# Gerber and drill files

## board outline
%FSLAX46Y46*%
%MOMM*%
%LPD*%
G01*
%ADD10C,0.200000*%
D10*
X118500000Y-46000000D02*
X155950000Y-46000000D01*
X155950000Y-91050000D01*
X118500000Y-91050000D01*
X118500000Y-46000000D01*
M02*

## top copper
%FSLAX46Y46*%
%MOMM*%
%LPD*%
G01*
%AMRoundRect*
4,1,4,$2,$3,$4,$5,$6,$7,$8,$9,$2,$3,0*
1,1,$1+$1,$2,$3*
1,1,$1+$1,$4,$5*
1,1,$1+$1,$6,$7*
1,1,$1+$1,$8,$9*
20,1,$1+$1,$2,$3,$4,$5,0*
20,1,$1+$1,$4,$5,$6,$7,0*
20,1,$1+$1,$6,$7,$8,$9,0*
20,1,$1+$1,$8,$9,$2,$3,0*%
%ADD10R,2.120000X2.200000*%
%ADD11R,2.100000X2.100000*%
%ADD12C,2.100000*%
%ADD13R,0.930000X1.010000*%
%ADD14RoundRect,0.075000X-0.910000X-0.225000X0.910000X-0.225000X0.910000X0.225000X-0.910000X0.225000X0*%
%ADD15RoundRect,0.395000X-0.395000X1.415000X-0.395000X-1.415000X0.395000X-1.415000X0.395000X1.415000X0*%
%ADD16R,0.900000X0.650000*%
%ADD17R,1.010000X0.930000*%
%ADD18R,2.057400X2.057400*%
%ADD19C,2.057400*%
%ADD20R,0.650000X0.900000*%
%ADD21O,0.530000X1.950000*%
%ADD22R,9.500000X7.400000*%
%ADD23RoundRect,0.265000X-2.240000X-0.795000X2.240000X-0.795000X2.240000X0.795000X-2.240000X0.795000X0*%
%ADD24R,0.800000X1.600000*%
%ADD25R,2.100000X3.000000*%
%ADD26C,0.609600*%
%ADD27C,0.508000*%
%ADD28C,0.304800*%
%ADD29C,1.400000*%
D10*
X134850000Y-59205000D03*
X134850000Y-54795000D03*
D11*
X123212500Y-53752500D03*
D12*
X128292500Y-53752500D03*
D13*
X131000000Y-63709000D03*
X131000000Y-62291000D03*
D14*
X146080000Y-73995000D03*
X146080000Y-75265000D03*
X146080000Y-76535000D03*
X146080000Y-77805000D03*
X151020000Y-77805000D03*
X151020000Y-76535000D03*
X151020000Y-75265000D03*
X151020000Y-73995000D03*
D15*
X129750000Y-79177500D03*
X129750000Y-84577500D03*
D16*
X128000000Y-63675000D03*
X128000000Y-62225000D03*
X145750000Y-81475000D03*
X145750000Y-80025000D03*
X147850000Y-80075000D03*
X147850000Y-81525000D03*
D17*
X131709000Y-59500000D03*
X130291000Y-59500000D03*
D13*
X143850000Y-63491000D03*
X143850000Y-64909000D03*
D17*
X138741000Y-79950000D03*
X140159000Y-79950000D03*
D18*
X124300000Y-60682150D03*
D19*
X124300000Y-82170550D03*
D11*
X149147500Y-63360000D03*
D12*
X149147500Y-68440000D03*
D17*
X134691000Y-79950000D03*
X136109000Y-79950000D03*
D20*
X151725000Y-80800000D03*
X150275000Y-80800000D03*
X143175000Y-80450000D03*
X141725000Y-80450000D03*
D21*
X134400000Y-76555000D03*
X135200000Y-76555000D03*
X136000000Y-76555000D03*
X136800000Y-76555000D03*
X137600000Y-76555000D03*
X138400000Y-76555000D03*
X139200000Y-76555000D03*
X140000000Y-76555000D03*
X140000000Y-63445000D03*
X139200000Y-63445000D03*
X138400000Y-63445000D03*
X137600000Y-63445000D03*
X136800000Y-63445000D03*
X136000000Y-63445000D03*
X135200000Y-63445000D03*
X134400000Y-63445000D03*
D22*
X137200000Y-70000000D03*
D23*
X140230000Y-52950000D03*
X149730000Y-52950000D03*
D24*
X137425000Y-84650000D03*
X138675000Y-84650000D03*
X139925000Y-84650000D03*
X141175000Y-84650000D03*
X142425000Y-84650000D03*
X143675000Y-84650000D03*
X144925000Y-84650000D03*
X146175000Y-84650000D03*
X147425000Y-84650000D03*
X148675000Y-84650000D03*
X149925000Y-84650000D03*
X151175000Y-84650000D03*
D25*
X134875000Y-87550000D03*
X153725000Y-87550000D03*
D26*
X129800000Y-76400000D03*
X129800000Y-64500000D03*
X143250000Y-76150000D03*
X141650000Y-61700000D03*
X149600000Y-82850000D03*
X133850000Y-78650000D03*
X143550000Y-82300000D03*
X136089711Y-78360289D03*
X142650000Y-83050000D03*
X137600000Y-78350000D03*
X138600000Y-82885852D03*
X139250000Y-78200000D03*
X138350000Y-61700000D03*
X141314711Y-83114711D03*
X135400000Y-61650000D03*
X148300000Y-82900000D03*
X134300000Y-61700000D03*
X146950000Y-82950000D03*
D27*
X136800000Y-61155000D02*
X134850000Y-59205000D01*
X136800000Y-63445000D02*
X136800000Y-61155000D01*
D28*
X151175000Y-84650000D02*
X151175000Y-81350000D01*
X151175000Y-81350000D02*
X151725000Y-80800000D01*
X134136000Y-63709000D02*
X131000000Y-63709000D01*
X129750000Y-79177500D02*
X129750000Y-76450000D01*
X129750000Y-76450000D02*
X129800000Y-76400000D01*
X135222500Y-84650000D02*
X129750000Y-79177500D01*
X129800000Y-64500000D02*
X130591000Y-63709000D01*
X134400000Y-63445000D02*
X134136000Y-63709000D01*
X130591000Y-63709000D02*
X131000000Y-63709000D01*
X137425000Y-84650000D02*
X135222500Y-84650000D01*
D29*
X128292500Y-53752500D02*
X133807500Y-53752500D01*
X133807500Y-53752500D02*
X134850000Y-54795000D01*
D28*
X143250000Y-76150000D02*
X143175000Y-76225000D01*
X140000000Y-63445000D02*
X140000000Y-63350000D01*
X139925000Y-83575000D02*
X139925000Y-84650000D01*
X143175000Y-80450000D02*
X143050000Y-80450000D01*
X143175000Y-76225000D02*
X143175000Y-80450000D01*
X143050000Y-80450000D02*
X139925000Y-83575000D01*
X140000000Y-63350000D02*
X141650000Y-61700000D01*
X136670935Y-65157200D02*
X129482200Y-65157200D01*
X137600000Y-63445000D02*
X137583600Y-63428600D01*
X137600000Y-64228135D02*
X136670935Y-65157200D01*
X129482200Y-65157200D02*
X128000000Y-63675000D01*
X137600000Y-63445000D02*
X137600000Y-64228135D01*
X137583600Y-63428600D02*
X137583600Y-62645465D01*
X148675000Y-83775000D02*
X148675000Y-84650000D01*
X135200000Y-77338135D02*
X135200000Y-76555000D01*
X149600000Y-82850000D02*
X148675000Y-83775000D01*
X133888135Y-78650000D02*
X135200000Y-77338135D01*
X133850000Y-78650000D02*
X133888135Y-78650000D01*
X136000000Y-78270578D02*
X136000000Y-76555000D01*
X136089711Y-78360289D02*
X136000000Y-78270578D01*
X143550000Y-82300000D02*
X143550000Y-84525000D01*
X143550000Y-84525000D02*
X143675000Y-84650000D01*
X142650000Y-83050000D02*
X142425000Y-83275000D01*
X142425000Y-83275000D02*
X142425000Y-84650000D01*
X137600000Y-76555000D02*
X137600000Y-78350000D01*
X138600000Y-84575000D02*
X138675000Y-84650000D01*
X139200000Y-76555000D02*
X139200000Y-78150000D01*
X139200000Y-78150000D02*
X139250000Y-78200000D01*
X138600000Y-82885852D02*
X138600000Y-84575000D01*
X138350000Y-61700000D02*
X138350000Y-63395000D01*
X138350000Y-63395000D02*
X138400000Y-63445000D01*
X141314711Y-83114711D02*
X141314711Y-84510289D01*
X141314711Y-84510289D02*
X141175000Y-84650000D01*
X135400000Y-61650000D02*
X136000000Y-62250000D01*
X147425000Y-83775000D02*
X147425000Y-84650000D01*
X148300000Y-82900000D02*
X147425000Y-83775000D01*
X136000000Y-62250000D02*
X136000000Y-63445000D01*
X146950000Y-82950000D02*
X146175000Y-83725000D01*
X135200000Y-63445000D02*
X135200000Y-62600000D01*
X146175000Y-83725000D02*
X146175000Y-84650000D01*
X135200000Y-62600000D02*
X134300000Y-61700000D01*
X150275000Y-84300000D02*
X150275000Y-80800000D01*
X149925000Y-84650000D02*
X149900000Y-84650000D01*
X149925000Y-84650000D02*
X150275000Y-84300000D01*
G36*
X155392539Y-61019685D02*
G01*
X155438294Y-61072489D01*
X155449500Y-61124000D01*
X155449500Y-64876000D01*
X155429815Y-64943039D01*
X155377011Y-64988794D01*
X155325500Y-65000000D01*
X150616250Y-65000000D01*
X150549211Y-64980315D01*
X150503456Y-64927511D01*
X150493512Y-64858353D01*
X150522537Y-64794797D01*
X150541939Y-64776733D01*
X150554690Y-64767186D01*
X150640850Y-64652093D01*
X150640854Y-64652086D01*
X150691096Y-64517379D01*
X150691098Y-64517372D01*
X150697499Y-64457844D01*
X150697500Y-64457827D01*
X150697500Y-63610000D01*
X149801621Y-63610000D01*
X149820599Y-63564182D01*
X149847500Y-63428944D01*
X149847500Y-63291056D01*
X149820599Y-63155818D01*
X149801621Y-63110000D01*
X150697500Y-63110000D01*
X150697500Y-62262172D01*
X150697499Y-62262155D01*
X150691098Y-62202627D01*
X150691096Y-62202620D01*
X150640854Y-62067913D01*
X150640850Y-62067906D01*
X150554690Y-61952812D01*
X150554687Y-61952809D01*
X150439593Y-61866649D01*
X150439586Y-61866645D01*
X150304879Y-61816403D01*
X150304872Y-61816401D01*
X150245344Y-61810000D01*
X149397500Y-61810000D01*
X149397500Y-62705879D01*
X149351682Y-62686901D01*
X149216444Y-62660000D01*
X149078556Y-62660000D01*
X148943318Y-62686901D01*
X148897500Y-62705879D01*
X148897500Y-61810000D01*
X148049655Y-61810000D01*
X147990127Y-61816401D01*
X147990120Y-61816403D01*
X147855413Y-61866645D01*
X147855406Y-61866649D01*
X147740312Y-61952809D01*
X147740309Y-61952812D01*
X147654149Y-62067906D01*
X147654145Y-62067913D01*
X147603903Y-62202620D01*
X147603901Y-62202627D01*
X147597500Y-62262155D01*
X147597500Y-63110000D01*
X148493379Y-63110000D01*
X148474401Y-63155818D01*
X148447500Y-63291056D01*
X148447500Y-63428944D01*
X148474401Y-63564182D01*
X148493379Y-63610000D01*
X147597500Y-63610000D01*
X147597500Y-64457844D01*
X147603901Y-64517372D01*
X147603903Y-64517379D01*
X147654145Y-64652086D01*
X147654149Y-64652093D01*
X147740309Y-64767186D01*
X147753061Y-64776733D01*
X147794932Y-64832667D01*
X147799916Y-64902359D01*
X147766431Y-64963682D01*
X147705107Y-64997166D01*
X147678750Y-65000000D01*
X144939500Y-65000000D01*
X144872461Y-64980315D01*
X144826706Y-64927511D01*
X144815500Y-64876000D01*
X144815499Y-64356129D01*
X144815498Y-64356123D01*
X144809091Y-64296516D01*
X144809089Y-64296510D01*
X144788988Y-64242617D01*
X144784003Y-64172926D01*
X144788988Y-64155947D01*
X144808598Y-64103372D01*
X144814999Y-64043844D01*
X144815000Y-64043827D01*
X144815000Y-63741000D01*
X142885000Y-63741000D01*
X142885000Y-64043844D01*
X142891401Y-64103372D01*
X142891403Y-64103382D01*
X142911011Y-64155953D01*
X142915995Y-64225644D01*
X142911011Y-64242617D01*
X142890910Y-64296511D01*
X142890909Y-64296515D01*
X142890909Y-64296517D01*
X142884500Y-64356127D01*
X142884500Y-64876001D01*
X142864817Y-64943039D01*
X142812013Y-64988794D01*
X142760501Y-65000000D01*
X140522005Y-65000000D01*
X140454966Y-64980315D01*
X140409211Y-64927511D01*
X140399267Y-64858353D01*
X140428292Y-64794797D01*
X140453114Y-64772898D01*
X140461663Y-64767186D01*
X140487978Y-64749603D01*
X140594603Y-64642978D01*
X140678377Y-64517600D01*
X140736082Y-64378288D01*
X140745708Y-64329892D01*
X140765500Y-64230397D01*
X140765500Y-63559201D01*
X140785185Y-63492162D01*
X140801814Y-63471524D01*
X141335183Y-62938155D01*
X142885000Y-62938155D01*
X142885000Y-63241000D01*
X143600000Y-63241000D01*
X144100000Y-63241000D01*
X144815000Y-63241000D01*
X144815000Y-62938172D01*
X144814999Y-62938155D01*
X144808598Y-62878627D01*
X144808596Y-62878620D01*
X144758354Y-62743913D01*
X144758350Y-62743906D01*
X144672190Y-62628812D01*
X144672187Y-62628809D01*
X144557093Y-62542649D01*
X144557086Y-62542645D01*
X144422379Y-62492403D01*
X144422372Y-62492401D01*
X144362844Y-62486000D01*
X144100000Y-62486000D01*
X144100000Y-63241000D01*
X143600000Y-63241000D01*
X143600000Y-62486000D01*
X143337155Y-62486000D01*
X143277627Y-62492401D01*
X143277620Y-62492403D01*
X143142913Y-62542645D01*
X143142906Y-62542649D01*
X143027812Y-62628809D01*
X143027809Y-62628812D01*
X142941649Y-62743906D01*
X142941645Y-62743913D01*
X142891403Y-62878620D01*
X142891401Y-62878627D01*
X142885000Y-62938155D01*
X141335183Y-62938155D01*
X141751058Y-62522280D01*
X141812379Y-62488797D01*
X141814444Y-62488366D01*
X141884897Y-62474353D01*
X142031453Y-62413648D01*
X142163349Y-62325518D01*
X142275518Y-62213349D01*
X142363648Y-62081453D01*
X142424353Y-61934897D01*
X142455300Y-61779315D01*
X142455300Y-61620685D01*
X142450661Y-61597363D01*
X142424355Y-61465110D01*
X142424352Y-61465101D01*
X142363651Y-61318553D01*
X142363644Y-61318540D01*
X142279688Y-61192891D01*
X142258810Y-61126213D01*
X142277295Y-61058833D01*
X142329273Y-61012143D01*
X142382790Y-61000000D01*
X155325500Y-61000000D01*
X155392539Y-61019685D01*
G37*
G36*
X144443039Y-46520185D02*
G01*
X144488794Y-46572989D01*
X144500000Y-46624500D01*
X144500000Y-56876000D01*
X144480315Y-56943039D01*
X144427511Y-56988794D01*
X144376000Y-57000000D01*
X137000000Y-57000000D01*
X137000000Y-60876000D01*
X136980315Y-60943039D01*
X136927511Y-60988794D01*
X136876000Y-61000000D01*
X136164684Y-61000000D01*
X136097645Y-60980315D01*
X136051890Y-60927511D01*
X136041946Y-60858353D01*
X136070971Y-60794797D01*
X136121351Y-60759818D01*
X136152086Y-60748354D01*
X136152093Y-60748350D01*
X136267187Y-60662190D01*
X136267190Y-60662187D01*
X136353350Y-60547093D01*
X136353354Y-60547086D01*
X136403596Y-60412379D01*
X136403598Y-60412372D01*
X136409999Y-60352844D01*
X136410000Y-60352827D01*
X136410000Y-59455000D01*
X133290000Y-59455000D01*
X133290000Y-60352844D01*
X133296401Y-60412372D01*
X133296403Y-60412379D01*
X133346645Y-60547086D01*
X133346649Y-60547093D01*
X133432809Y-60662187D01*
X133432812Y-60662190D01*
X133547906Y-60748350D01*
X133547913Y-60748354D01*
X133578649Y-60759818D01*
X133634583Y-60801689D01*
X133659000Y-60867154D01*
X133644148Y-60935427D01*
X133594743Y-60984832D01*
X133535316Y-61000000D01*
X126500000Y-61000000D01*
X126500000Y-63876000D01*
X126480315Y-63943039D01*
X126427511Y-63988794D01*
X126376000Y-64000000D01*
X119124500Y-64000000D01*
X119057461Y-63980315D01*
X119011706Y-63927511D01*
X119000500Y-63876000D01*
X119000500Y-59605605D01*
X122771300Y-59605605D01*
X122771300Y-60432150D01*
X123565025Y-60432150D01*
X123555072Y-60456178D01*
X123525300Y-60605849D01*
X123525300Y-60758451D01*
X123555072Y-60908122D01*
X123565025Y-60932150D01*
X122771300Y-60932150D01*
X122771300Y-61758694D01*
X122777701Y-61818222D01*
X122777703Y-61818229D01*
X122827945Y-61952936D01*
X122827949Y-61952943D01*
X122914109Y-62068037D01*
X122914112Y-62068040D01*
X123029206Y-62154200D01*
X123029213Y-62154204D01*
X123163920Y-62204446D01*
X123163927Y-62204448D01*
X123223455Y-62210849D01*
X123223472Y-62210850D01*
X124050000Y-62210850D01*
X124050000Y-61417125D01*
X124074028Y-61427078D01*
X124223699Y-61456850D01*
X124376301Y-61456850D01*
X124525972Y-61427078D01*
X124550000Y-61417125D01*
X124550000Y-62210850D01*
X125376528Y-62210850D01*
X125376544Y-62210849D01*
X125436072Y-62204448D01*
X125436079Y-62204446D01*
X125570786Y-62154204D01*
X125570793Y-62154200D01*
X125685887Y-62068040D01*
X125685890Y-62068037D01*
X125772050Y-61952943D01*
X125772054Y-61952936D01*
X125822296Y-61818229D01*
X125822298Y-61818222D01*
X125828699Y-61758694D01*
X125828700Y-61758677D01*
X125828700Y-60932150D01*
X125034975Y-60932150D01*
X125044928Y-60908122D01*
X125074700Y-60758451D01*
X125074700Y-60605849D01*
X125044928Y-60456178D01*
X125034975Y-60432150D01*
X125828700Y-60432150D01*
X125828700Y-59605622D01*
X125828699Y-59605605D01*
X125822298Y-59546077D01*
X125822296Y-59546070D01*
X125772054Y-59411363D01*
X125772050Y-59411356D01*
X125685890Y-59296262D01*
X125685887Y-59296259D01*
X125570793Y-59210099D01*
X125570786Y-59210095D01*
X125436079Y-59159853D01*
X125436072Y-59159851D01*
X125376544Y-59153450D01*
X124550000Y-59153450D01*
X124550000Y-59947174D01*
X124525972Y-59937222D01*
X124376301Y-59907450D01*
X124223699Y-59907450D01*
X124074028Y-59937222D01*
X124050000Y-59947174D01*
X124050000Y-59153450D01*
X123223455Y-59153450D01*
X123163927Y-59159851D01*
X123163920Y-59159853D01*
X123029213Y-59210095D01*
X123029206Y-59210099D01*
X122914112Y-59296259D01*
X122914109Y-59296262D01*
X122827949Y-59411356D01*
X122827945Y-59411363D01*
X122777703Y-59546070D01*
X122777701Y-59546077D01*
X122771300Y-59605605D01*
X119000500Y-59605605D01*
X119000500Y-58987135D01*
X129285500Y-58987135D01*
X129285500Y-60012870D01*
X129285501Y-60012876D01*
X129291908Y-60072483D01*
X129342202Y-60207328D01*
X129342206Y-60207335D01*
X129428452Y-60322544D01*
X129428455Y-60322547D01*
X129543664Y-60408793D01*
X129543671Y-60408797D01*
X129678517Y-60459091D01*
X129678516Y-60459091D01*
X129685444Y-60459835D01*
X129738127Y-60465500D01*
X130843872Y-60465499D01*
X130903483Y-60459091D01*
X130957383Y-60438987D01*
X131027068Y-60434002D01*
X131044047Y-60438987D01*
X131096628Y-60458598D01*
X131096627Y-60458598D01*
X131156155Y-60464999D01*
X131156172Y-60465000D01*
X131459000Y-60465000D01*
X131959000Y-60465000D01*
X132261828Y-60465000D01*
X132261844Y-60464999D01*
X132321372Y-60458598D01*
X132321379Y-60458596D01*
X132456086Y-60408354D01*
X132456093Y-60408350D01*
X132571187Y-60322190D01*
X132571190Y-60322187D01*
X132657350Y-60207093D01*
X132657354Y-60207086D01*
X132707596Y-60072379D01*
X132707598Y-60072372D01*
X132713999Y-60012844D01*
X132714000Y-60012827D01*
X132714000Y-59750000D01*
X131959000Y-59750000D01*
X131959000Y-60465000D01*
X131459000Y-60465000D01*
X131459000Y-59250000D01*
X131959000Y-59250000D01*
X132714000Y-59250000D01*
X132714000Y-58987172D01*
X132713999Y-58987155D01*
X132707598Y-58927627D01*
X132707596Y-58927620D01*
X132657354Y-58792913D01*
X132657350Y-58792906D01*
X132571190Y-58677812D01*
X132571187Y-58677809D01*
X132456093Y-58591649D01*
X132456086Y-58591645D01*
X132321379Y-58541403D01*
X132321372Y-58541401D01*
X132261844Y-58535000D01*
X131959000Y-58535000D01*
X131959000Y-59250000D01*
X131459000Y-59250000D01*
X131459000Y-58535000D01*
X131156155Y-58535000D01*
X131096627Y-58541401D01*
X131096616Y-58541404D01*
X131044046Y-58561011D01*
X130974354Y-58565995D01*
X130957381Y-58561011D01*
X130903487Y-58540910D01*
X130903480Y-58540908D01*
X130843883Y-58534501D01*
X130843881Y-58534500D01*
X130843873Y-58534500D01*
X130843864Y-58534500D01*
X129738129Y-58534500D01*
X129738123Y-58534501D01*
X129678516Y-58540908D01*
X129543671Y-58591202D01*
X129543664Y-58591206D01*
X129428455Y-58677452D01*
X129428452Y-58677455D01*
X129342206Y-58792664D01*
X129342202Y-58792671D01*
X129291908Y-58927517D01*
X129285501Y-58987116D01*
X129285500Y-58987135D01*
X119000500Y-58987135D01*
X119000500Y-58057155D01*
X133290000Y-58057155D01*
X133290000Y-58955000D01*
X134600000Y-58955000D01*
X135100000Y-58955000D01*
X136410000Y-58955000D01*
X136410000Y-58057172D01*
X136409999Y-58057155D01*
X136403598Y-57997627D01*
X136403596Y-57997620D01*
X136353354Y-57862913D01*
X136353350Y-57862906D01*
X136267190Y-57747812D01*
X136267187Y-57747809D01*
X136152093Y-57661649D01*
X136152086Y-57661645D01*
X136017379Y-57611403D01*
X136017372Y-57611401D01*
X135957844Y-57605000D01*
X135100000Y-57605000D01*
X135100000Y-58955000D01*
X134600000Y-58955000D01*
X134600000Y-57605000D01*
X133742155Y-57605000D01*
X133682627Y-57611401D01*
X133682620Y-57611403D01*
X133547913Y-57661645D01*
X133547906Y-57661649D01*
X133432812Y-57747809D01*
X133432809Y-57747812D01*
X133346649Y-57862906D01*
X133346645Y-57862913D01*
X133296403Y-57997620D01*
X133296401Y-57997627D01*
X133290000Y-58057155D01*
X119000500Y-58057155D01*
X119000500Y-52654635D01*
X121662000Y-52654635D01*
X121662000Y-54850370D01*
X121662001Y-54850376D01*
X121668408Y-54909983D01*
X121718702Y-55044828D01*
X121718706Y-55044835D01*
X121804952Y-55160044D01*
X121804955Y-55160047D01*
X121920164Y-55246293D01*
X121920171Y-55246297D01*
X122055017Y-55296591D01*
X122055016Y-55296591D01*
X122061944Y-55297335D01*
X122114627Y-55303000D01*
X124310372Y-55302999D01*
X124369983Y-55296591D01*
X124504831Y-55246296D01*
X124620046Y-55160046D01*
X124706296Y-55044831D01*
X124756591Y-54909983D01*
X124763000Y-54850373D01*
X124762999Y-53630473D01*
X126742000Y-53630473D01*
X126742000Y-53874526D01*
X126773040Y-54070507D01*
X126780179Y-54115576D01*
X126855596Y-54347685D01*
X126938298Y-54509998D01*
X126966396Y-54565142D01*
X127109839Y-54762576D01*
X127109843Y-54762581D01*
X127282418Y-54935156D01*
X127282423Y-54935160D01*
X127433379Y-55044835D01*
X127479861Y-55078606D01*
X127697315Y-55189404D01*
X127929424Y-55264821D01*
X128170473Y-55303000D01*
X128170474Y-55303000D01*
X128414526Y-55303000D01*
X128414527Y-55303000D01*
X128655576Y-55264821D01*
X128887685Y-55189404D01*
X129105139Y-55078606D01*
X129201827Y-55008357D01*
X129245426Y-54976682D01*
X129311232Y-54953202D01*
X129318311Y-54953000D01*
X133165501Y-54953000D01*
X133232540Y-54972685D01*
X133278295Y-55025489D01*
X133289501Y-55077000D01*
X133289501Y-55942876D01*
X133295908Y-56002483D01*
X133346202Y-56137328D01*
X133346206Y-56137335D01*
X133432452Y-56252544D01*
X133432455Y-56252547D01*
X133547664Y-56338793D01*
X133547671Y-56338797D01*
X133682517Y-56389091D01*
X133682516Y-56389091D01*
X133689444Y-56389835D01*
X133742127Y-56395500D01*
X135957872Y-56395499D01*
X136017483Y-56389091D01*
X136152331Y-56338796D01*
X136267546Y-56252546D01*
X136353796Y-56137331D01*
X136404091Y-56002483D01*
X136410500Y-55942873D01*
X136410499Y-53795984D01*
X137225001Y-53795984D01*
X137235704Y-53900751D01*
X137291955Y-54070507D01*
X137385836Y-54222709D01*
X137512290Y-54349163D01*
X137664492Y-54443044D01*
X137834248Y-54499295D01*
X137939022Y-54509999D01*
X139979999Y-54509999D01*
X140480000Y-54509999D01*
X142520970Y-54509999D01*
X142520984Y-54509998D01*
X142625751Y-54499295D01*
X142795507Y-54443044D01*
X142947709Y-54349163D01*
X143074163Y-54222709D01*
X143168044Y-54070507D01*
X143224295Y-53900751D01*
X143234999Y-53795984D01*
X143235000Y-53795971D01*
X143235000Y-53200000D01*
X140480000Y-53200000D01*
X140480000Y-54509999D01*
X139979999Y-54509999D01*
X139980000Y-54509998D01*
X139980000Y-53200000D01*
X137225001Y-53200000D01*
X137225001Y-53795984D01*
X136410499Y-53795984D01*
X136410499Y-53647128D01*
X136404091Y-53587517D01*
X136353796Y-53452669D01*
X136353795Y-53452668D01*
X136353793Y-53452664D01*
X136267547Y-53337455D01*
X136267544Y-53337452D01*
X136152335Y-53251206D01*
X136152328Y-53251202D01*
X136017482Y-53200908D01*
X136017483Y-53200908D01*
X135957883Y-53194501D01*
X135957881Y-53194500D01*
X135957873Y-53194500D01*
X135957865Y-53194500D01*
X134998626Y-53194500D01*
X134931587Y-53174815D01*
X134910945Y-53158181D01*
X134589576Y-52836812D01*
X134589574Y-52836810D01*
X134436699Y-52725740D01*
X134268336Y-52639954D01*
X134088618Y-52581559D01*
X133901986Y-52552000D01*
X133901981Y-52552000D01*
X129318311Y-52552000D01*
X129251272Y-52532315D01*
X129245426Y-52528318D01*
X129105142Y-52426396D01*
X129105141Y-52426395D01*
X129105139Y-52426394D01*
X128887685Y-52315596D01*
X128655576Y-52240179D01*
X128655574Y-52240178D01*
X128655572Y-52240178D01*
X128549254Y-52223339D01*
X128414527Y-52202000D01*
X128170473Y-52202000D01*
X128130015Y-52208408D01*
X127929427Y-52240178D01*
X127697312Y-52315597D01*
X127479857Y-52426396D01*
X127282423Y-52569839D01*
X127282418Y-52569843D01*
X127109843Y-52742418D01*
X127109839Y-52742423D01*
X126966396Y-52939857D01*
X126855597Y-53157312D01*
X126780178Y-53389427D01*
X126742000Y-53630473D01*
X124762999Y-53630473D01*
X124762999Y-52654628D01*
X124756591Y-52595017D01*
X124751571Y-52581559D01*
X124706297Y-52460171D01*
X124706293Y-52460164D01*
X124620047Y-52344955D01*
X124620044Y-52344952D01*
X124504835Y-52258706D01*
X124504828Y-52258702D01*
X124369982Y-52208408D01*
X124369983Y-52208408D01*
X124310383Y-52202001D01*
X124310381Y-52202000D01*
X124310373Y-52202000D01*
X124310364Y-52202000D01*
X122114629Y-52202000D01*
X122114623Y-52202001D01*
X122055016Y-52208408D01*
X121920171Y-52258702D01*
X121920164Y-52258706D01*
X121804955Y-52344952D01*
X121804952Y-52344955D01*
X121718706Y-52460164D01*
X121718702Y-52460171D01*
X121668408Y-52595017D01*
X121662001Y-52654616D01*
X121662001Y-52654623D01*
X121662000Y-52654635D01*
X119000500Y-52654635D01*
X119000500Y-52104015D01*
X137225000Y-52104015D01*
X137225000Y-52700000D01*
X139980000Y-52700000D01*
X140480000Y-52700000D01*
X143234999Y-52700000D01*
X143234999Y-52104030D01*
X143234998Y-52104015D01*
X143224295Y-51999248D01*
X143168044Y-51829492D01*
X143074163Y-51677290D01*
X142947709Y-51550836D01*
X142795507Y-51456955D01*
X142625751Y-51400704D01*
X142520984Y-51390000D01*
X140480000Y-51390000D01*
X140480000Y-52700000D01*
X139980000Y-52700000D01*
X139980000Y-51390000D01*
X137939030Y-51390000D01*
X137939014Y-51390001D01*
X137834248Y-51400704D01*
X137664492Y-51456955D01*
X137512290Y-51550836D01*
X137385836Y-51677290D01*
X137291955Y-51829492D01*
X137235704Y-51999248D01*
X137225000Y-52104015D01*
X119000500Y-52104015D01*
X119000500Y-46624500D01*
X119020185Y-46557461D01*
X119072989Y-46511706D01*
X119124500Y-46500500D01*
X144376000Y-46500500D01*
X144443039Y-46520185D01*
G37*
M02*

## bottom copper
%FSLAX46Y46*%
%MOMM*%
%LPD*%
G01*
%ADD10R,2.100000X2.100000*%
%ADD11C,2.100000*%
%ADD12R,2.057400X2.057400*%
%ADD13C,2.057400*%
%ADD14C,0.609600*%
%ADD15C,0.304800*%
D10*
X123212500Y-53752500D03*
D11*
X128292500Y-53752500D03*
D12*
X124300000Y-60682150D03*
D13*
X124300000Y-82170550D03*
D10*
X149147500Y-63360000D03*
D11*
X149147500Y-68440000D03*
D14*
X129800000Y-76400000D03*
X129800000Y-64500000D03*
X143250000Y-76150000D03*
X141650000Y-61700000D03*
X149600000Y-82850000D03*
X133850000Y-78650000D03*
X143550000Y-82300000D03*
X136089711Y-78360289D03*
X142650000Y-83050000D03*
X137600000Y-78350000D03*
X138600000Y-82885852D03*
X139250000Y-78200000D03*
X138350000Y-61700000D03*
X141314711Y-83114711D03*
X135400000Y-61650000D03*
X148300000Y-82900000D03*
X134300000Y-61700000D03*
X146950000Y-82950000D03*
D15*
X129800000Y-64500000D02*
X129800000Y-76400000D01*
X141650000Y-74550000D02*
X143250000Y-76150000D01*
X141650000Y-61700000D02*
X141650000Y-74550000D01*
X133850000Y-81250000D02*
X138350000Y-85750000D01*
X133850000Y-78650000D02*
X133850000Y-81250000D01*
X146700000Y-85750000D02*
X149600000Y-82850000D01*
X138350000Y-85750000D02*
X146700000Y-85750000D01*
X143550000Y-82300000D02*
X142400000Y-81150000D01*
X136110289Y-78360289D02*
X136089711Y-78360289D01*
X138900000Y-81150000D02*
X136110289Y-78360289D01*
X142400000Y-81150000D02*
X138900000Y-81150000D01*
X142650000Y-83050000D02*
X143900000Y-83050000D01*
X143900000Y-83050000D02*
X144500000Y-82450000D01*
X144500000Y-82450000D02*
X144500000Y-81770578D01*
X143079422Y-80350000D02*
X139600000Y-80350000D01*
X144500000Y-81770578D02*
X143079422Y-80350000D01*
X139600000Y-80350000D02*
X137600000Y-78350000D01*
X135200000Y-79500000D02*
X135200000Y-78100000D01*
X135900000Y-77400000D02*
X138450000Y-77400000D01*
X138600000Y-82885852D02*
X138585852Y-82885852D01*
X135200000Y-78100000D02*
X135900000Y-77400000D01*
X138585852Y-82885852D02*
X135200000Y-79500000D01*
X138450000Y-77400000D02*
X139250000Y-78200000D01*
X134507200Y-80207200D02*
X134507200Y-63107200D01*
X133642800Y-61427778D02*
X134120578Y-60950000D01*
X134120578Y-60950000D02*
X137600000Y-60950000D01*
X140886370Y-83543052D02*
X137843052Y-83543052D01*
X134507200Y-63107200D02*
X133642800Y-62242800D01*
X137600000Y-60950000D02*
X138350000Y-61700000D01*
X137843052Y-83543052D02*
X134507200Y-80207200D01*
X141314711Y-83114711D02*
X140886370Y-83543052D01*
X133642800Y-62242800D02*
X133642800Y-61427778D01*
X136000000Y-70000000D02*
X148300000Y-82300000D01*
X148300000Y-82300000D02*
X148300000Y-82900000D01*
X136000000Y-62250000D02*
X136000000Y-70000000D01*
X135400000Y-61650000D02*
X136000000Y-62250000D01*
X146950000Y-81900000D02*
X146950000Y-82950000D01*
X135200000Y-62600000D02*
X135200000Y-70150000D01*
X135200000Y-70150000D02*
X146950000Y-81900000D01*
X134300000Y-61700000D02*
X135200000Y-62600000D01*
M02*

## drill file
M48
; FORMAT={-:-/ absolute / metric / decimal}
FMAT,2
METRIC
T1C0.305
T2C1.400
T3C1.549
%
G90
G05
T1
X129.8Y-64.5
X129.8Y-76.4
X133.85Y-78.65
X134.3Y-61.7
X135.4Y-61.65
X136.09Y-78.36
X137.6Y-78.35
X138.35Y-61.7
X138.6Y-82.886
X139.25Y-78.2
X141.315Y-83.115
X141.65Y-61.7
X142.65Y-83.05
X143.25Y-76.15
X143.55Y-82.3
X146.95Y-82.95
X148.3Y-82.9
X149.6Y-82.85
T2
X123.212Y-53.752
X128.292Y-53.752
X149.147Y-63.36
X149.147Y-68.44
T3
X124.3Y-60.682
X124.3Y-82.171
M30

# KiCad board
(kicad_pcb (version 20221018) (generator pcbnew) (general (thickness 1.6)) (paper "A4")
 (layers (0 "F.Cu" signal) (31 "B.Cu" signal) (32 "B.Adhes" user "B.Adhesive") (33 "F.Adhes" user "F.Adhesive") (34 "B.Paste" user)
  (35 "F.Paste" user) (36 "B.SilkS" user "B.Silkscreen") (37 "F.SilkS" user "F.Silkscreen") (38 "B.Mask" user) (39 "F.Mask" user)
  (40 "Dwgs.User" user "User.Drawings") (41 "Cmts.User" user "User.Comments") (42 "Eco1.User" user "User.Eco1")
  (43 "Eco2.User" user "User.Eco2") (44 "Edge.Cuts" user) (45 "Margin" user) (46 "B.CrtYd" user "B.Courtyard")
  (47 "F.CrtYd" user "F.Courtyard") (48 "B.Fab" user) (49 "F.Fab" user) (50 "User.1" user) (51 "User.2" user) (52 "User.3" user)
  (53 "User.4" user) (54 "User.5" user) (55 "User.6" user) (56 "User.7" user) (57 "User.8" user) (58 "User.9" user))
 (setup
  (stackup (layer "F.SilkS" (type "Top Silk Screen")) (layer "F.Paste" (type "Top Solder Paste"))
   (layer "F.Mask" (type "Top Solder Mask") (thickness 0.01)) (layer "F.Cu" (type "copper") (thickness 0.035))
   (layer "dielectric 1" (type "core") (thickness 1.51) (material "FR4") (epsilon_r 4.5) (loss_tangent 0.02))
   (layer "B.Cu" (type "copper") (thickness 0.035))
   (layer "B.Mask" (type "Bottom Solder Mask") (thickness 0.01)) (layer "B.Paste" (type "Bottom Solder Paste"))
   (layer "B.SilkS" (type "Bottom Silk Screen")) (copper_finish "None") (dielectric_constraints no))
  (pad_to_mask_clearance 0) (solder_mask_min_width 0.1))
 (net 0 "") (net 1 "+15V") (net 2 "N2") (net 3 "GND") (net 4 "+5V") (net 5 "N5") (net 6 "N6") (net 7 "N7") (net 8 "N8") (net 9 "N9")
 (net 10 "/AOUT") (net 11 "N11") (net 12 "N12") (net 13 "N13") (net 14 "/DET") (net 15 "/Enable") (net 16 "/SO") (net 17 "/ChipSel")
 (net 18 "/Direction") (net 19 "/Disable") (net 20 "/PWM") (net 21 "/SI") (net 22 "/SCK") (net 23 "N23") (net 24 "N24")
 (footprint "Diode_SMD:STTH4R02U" (layer "F.Cu") (at 134.85 57 90)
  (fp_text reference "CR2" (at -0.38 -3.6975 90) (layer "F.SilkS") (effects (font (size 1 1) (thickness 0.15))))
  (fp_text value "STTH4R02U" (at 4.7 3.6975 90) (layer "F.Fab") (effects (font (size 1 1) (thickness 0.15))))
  (pad "1" smd rect (at -2.205 0 90) (size 2.2 2.12) (layers "F.Cu" "F.Paste" "F.Mask") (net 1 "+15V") (solder_mask_margin 0.102))
  (pad "2" smd rect (at 2.205 0 90) (size 2.2 2.12) (layers "F.Cu" "F.Paste" "F.Mask") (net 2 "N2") (solder_mask_margin 0.102)))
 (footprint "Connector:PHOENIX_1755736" (layer "F.Cu") (at 119.6725 57.6225)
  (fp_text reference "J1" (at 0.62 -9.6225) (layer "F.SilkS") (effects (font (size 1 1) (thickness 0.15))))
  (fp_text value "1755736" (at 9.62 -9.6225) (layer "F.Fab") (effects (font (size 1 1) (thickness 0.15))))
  (pad "1" thru_hole rect (at 3.54 -3.87) (size 2.1 2.1) (drill 1.4) (layers "*.Cu" "*.Mask") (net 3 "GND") (solder_mask_margin 0.102))
  (pad "2" thru_hole circle (at 8.62 -3.87) (size 2.1 2.1) (drill 1.4) (layers "*.Cu" "*.Mask") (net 2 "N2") (solder_mask_margin 0.102)))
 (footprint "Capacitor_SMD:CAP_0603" (layer "F.Cu") (at 131 63 90)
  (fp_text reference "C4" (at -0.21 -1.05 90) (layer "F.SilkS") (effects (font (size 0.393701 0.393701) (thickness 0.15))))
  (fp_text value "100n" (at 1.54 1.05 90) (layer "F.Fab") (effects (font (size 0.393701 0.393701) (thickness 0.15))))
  (pad "1" smd rect (at -0.709 0 90) (size 1.01 0.93) (layers "F.Cu" "F.Paste" "F.Mask") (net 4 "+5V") (solder_mask_margin 0.102))
  (pad "2" smd rect (at 0.709 0 90) (size 1.01 0.93) (layers "F.Cu" "F.Paste" "F.Mask") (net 3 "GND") (solder_mask_margin 0.102)))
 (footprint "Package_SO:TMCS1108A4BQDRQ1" (layer "F.Cu") (at 148.55 75.9)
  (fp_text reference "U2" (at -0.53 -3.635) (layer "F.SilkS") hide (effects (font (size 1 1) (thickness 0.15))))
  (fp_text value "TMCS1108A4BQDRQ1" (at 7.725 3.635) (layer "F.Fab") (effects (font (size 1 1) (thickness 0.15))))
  (pad "1" smd roundrect (at -2.47 -1.905) (size 1.97 0.6) (layers "F.Cu" "F.Paste" "F.Mask") (roundrect_rratio 0.125) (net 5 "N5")
   (solder_mask_margin 0.102))
  (pad "2" smd roundrect (at -2.47 -0.635) (size 1.97 0.6) (layers "F.Cu" "F.Paste" "F.Mask") (roundrect_rratio 0.125) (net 5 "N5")
   (solder_mask_margin 0.102))
  (pad "3" smd roundrect (at -2.47 0.635) (size 1.97 0.6) (layers "F.Cu" "F.Paste" "F.Mask") (roundrect_rratio 0.125) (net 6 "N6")
   (solder_mask_margin 0.102))
  (pad "4" smd roundrect (at -2.47 1.905) (size 1.97 0.6) (layers "F.Cu" "F.Paste" "F.Mask") (roundrect_rratio 0.125) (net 6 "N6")
   (solder_mask_margin 0.102))
  (pad "5" smd roundrect (at 2.47 1.905) (size 1.97 0.6) (layers "F.Cu" "F.Paste" "F.Mask") (roundrect_rratio 0.125) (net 3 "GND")
   (solder_mask_margin 0.102))
  (pad "6" smd roundrect (at 2.47 0.635) (size 1.97 0.6) (layers "F.Cu" "F.Paste" "F.Mask") (roundrect_rratio 0.125) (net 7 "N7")
   (solder_mask_margin 0.102))
  (pad "7" smd roundrect (at 2.47 -0.635) (size 1.97 0.6) (layers "F.Cu" "F.Paste" "F.Mask") (roundrect_rratio 0.125) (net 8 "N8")
   (solder_mask_margin 0.102))
  (pad "8" smd roundrect (at 2.47 -1.905) (size 1.97 0.6) (layers "F.Cu" "F.Paste" "F.Mask") (roundrect_rratio 0.125) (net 4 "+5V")
   (solder_mask_margin 0.102)))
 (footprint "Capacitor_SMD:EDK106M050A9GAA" (layer "F.Cu") (at 129.75 81.8775 -90)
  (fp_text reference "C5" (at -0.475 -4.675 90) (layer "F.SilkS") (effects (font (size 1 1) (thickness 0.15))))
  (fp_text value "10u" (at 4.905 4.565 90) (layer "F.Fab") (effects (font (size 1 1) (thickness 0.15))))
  (pad "1" smd roundrect (at -2.7 0 270) (size 3.62 1.58) (layers "F.Cu" "F.Paste" "F.Mask") (roundrect_rratio 0.25) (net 4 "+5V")
   (solder_mask_margin 0.102))
  (pad "2" smd roundrect (at 2.7 0 270) (size 3.62 1.58) (layers "F.Cu" "F.Paste" "F.Mask") (roundrect_rratio 0.25) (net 3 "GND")
   (solder_mask_margin 0.102)))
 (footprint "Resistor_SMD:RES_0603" (layer "F.Cu") (at 128 62.95 90)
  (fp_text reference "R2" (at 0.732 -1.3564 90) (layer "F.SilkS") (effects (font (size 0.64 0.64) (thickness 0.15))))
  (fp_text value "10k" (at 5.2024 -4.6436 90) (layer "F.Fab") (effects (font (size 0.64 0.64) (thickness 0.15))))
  (pad "1" smd rect (at -0.725 0 90) (size 0.65 0.9) (layers "F.Cu" "F.Paste" "F.Mask") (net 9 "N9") (solder_mask_margin 0.102))
  (pad "2" smd rect (at 0.725 0 90) (size 0.65 0.9) (layers "F.Cu" "F.Paste" "F.Mask") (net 3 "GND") (solder_mask_margin 0.102)))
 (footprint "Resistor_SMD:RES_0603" (layer "F.Cu") (at 145.75 80.75 90)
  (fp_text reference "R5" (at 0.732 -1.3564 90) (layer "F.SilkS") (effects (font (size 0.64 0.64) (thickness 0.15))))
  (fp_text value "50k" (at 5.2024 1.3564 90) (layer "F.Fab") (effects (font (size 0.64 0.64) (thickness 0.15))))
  (pad "1" smd rect (at -0.725 0 90) (size 0.65 0.9) (layers "F.Cu" "F.Paste" "F.Mask") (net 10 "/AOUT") (solder_mask_margin 0.102))
  (pad "2" smd rect (at 0.725 0 90) (size 0.65 0.9) (layers "F.Cu" "F.Paste" "F.Mask") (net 3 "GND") (solder_mask_margin 0.102)))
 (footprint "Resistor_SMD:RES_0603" (layer "F.Cu") (at 147.85 80.8 -90)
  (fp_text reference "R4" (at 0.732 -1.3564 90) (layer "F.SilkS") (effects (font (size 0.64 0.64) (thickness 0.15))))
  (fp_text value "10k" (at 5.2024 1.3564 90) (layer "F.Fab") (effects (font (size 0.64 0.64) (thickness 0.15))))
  (pad "1" smd rect (at -0.725 0 270) (size 0.65 0.9) (layers "F.Cu" "F.Paste" "F.Mask") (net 8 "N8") (solder_mask_margin 0.102))
  (pad "2" smd rect (at 0.725 0 270) (size 0.65 0.9) (layers "F.Cu" "F.Paste" "F.Mask") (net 10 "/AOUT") (solder_mask_margin 0.102)))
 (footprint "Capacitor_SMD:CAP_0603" (layer "F.Cu") (at 131 59.5 180)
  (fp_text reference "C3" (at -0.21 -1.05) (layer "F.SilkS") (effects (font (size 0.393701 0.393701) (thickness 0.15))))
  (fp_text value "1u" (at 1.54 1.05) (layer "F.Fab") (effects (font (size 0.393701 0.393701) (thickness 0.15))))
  (pad "1" smd rect (at -0.709 0 180) (size 1.01 0.93) (layers "F.Cu" "F.Paste" "F.Mask") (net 1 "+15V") (solder_mask_margin 0.102))
  (pad "2" smd rect (at 0.709 0 180) (size 1.01 0.93) (layers "F.Cu" "F.Paste" "F.Mask") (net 3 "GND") (solder_mask_margin 0.102)))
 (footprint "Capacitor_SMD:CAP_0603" (layer "F.Cu") (at 143.85 64.2 -90)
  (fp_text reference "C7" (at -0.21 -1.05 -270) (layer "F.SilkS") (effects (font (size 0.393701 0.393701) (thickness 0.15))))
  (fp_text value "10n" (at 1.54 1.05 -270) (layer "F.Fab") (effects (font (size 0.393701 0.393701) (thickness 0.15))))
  (pad "1" smd rect (at -0.709 0 270) (size 1.01 0.93) (layers "F.Cu" "F.Paste" "F.Mask") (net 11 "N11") (solder_mask_margin 0.102))
  (pad "2" smd rect (at 0.709 0 270) (size 1.01 0.93) (layers "F.Cu" "F.Paste" "F.Mask") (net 3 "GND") (solder_mask_margin 0.102)))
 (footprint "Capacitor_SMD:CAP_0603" (layer "F.Cu") (at 139.45 79.95)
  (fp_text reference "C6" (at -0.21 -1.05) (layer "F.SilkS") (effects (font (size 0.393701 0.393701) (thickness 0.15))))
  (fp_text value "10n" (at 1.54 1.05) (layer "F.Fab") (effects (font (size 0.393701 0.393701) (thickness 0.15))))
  (pad "1" smd rect (at -0.709 0) (size 1.01 0.93) (layers "F.Cu" "F.Paste" "F.Mask") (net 5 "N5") (solder_mask_margin 0.102))
  (pad "2" smd rect (at 0.709 0) (size 1.01 0.93) (layers "F.Cu" "F.Paste" "F.Mask") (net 3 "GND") (solder_mask_margin 0.102)))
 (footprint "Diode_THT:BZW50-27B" (layer "F.Cu") (at 124.3 60.68215 -90)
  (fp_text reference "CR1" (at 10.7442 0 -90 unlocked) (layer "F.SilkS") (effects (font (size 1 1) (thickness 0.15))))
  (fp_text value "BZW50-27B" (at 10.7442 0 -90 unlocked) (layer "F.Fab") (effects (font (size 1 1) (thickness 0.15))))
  (pad "1" thru_hole rect (at 0 0 270) (size 2.0574 2.0574) (drill 1.5494) (layers "*.Cu" "*.Mask") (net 1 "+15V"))
  (pad "2" thru_hole circle (at 21.4884 0 270) (size 2.0574 2.0574) (drill 1.5494) (layers "*.Cu" "*.Mask") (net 3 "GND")))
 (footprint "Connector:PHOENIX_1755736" (layer "F.Cu") (at 145.2775 59.82 -90)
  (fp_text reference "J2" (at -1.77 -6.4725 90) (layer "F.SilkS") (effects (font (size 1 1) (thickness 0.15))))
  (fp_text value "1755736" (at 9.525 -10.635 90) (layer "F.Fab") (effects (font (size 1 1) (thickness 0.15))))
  (pad "1" thru_hole rect (at 3.54 -3.87 270) (size 2.1 2.1) (drill 1.4) (layers "*.Cu" "*.Mask") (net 11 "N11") (solder_mask_margin 0.102))
  (pad "2" thru_hole circle (at 8.62 -3.87 270) (size 2.1 2.1) (drill 1.4) (layers "*.Cu" "*.Mask") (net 6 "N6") (solder_mask_margin 0.102)))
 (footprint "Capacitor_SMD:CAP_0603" (layer "F.Cu") (at 135.4 79.95)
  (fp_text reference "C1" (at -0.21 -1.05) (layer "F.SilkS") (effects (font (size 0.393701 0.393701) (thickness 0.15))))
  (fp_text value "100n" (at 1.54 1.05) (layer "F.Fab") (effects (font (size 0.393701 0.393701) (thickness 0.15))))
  (pad "1" smd rect (at -0.709 0) (size 1.01 0.93) (layers "F.Cu" "F.Paste" "F.Mask") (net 1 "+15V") (solder_mask_margin 0.102))
  (pad "2" smd rect (at 0.709 0) (size 1.01 0.93) (layers "F.Cu" "F.Paste" "F.Mask") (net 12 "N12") (solder_mask_margin 0.102)))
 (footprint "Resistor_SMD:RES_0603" (layer "F.Cu") (at 151 80.8 180)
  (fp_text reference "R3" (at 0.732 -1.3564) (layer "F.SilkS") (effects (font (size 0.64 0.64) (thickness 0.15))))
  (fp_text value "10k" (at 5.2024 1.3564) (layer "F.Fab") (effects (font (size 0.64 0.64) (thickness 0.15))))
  (pad "1" smd rect (at -0.725 0 180) (size 0.65 0.9) (layers "F.Cu" "F.Paste" "F.Mask") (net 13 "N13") (solder_mask_margin 0.102))
  (pad "2" smd rect (at 0.725 0 180) (size 0.65 0.9) (layers "F.Cu" "F.Paste" "F.Mask") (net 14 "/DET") (solder_mask_margin 0.102)))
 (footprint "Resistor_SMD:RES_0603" (layer "F.Cu") (at 142.45 80.45 180)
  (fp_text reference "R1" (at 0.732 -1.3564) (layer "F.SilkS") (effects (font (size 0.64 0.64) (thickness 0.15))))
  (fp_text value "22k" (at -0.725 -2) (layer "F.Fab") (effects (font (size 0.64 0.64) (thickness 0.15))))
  (pad "1" smd rect (at -0.725 0 180) (size 0.65 0.9) (layers "F.Cu" "F.Paste" "F.Mask") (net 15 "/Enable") (solder_mask_margin 0.102))
  (pad "2" smd rect (at 0.725 0 180) (size 0.65 0.9) (layers "F.Cu" "F.Paste" "F.Mask") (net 3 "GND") (solder_mask_margin 0.102)))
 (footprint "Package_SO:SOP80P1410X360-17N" (layer "F.Cu") (at 137.2 70 90)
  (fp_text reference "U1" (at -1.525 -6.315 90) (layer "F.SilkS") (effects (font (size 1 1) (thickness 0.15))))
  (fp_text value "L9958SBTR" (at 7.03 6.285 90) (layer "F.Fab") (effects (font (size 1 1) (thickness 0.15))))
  (pad "1" smd oval (at -6.555 -2.8 90) (size 1.95 0.53) (layers "F.Cu" "F.Paste" "F.Mask") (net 3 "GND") (solder_mask_margin 0.102))
  (pad "2" smd oval (at -6.555 -2 90) (size 1.95 0.53) (layers "F.Cu" "F.Paste" "F.Mask") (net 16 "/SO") (solder_mask_margin 0.102))
  (pad "3" smd oval (at -6.555 -1.2 90) (size 1.95 0.53) (layers "F.Cu" "F.Paste" "F.Mask") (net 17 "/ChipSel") (solder_mask_margin 0.102))
  (pad "4" smd oval (at -6.555 -0.4 90) (size 1.95 0.53) (layers "F.Cu" "F.Paste" "F.Mask") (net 12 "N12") (solder_mask_margin 0.102))
  (pad "5" smd oval (at -6.555 0.4 90) (size 1.95 0.53) (layers "F.Cu" "F.Paste" "F.Mask") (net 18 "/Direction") (solder_mask_margin 0.102))
  (pad "6" smd oval (at -6.555 1.2 90) (size 1.95 0.53) (layers "F.Cu" "F.Paste" "F.Mask") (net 5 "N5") (solder_mask_margin 0.102))
  (pad "7" smd oval (at -6.555 2 90) (size 1.95 0.53) (layers "F.Cu" "F.Paste" "F.Mask") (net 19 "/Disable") (solder_mask_margin 0.102))
  (pad "8" smd oval (at -6.555 2.8 90) (size 1.95 0.53) (layers "F.Cu" "F.Paste" "F.Mask") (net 3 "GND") (solder_mask_margin 0.102))
  (pad "9" smd oval (at 6.555 2.8 90) (size 1.95 0.53) (layers "F.Cu" "F.Paste" "F.Mask") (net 15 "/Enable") (solder_mask_margin 0.102))
  (pad "10" smd oval (at 6.555 2 90) (size 1.95 0.53) (layers "F.Cu" "F.Paste" "F.Mask") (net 11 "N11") (solder_mask_margin 0.102))
  (pad "11" smd oval (at 6.555 1.2 90) (size 1.95 0.53) (layers "F.Cu" "F.Paste" "F.Mask") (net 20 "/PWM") (solder_mask_margin 0.102))
  (pad "12" smd oval (at 6.555 0.4 90) (size 1.95 0.53) (layers "F.Cu" "F.Paste" "F.Mask") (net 9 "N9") (solder_mask_margin 0.102))
  (pad "13" smd oval (at 6.555 -0.4 90) (size 1.95 0.53) (layers "F.Cu" "F.Paste" "F.Mask") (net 1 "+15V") (solder_mask_margin 0.102))
  (pad "14" smd oval (at 6.555 -1.2 90) (size 1.95 0.53) (layers "F.Cu" "F.Paste" "F.Mask") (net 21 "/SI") (solder_mask_margin 0.102))
  (pad "15" smd oval (at 6.555 -2 90) (size 1.95 0.53) (layers "F.Cu" "F.Paste" "F.Mask") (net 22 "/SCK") (solder_mask_margin 0.102))
  (pad "16" smd oval (at 6.555 -2.8 90) (size 1.95 0.53) (layers "F.Cu" "F.Paste" "F.Mask") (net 4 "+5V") (solder_mask_margin 0.102))
  (pad "17" smd rect (at 0 0 90) (size 7.4 9.5) (layers "F.Cu" "F.Mask") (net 3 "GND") (solder_mask_margin 0.102)))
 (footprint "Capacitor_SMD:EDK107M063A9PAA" (layer "F.Cu") (at 144.98 52.95)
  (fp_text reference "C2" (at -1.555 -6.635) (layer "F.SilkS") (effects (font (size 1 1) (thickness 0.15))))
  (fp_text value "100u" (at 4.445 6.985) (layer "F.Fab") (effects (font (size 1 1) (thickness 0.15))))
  (pad "1" smd roundrect (at -4.75 0) (size 5.01 2.12) (layers "F.Cu" "F.Paste" "F.Mask") (roundrect_rratio 0.125) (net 1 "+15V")
   (solder_mask_margin 0.102))
  (pad "2" smd roundrect (at 4.75 0) (size 5.01 2.12) (layers "F.Cu" "F.Paste" "F.Mask") (roundrect_rratio 0.125) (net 3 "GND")
   (solder_mask_margin 0.102)))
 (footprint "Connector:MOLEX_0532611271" (layer "F.Cu") (at 144.3 87.55)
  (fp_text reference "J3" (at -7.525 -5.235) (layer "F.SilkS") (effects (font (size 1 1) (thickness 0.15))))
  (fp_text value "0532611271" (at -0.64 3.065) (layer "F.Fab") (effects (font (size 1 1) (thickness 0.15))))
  (pad "1" smd rect (at -6.875 -2.9) (size 0.8 1.6) (layers "F.Cu" "F.Paste" "F.Mask") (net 4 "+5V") (solder_mask_margin 0.0762))
  (pad "2" smd rect (at -5.625 -2.9) (size 0.8 1.6) (layers "F.Cu" "F.Paste" "F.Mask") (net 19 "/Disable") (solder_mask_margin 0.0762))
  (pad "3" smd rect (at -4.375 -2.9) (size 0.8 1.6) (layers "F.Cu" "F.Paste" "F.Mask") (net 15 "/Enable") (solder_mask_margin 0.0762))
  (pad "4" smd rect (at -3.125 -2.9) (size 0.8 1.6) (layers "F.Cu" "F.Paste" "F.Mask") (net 20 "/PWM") (solder_mask_margin 0.0762))
  (pad "5" smd rect (at -1.875 -2.9) (size 0.8 1.6) (layers "F.Cu" "F.Paste" "F.Mask") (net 18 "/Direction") (solder_mask_margin 0.0762))
  (pad "6" smd rect (at -0.625 -2.9) (size 0.8 1.6) (layers "F.Cu" "F.Paste" "F.Mask") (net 17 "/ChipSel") (solder_mask_margin 0.0762))
  (pad "7" smd rect (at 0.625 -2.9) (size 0.8 1.6) (layers "F.Cu" "F.Paste" "F.Mask") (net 10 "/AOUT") (solder_mask_margin 0.0762))
  (pad "8" smd rect (at 1.875 -2.9) (size 0.8 1.6) (layers "F.Cu" "F.Paste" "F.Mask") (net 22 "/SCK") (solder_mask_margin 0.0762))
  (pad "9" smd rect (at 3.125 -2.9) (size 0.8 1.6) (layers "F.Cu" "F.Paste" "F.Mask") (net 21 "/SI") (solder_mask_margin 0.0762))
  (pad "10" smd rect (at 4.375 -2.9) (size 0.8 1.6) (layers "F.Cu" "F.Paste" "F.Mask") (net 16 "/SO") (solder_mask_margin 0.0762))
  (pad "11" smd rect (at 5.625 -2.9) (size 0.8 1.6) (layers "F.Cu" "F.Paste" "F.Mask") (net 14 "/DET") (solder_mask_margin 0.0762))
  (pad "12" smd rect (at 6.875 -2.9) (size 0.8 1.6) (layers "F.Cu" "F.Paste" "F.Mask") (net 13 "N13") (solder_mask_margin 0.0762))
  (pad "S1" smd rect (at -9.425 0) (size 2.1 3) (layers "F.Cu" "F.Paste" "F.Mask") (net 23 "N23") (solder_mask_margin 0.0762))
  (pad "S2" smd rect (at 9.425 0) (size 2.1 3) (layers "F.Cu" "F.Paste" "F.Mask") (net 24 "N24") (solder_mask_margin 0.0762)))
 (gr_rect (start 118.5 46) (end 155.95 91.05) (stroke (width 0.2) (type default)) (fill none) (layer "Edge.Cuts"))
 (segment (start 136.8 61.155) (end 134.85 59.205) (width 0.508) (layer "F.Cu") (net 1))
 (segment (start 136.8 63.445) (end 136.8 61.155) (width 0.508) (layer "F.Cu") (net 1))
 (segment (start 151.175 84.65) (end 151.175 81.35) (width 0.3048) (layer "F.Cu") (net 13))
 (segment (start 151.175 81.35) (end 151.725 80.8) (width 0.3048) (layer "F.Cu") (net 13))
 (segment (start 134.136 63.709) (end 131 63.709) (width 0.3048) (layer "F.Cu") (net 4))
 (segment (start 129.75 79.1775) (end 129.75 76.45) (width 0.3048) (layer "F.Cu") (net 4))
 (segment (start 129.75 76.45) (end 129.8 76.4) (width 0.3048) (layer "F.Cu") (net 4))
 (segment (start 135.2225 84.65) (end 129.75 79.1775) (width 0.3048) (layer "F.Cu") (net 4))
 (segment (start 129.8 64.5) (end 130.591 63.709) (width 0.3048) (layer "F.Cu") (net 4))
 (segment (start 134.4 63.445) (end 134.136 63.709) (width 0.3048) (layer "F.Cu") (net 4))
 (segment (start 130.591 63.709) (end 131 63.709) (width 0.3048) (layer "F.Cu") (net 4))
 (segment (start 137.425 84.65) (end 135.2225 84.65) (width 0.3048) (layer "F.Cu") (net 4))
 (via (at 129.8 76.4) (size 0.6096) (drill 0.3048) (layers "F.Cu" "B.Cu") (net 4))
 (via (at 129.8 64.5) (size 0.6096) (drill 0.3048) (layers "F.Cu" "B.Cu") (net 4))
 (segment (start 129.8 64.5) (end 129.8 76.4) (width 0.3048) (layer "B.Cu") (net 4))
 (segment (start 128.2925 53.7525) (end 133.8075 53.7525) (width 1.4) (layer "F.Cu") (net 2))
 (segment (start 133.8075 53.7525) (end 134.85 54.795) (width 1.4) (layer "F.Cu") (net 2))
 (segment (start 143.25 76.15) (end 143.175 76.225) (width 0.3048) (layer "F.Cu") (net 15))
 (segment (start 140 63.445) (end 140 63.35) (width 0.3048) (layer "F.Cu") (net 15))
 (segment (start 139.925 83.575) (end 139.925 84.65) (width 0.3048) (layer "F.Cu") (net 15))
 (segment (start 143.175 80.45) (end 143.05 80.45) (width 0.3048) (layer "F.Cu") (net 15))
 (segment (start 143.175 76.225) (end 143.175 80.45) (width 0.3048) (layer "F.Cu") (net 15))
 (segment (start 143.05 80.45) (end 139.925 83.575) (width 0.3048) (layer "F.Cu") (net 15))
 (segment (start 140 63.35) (end 141.65 61.7) (width 0.3048) (layer "F.Cu") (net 15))
 (via (at 143.25 76.15) (size 0.6096) (drill 0.3048) (layers "F.Cu" "B.Cu") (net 15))
 (via (at 141.65 61.7) (size 0.6096) (drill 0.3048) (layers "F.Cu" "B.Cu") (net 15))
 (segment (start 141.65 74.55) (end 143.25 76.15) (width 0.3048) (layer "B.Cu") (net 15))
 (segment (start 141.65 61.7) (end 141.65 74.55) (width 0.3048) (layer "B.Cu") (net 15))
 (segment (start 136.670935 65.1572) (end 129.4822 65.1572) (width 0.3048) (layer "F.Cu") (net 9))
 (segment (start 137.6 63.445) (end 137.5836 63.4286) (width 0.3048) (layer "F.Cu") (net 9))
 (segment (start 137.6 64.228135) (end 136.670935 65.1572) (width 0.3048) (layer "F.Cu") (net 9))
 (segment (start 129.4822 65.1572) (end 128 63.675) (width 0.3048) (layer "F.Cu") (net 9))
 (segment (start 137.6 63.445) (end 137.6 64.228135) (width 0.3048) (layer "F.Cu") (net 9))
 (segment (start 137.5836 63.4286) (end 137.5836 62.645465) (width 0.3048) (layer "F.Cu") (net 9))
 (segment (start 148.675 83.775) (end 148.675 84.65) (width 0.3048) (layer "F.Cu") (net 16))
 (segment (start 135.2 77.338135) (end 135.2 76.555) (width 0.3048) (layer "F.Cu") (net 16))
 (segment (start 149.6 82.85) (end 148.675 83.775) (width 0.3048) (layer "F.Cu") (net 16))
 (segment (start 133.888135 78.65) (end 135.2 77.338135) (width 0.3048) (layer "F.Cu") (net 16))
 (segment (start 133.85 78.65) (end 133.888135 78.65) (width 0.3048) (layer "F.Cu") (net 16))
 (via (at 149.6 82.85) (size 0.6096) (drill 0.3048) (layers "F.Cu" "B.Cu") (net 16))
 (via (at 133.85 78.65) (size 0.6096) (drill 0.3048) (layers "F.Cu" "B.Cu") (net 16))
 (segment (start 133.85 81.25) (end 138.35 85.75) (width 0.3048) (layer "B.Cu") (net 16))
 (segment (start 133.85 78.65) (end 133.85 81.25) (width 0.3048) (layer "B.Cu") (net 16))
 (segment (start 146.7 85.75) (end 149.6 82.85) (width 0.3048) (layer "B.Cu") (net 16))
 (segment (start 138.35 85.75) (end 146.7 85.75) (width 0.3048) (layer "B.Cu") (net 16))
 (segment (start 136 78.270578) (end 136 76.555) (width 0.3048) (layer "F.Cu") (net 17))
 (segment (start 136.089711 78.360289) (end 136 78.270578) (width 0.3048) (layer "F.Cu") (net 17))
 (segment (start 143.55 82.3) (end 143.55 84.525) (width 0.3048) (layer "F.Cu") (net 17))
 (segment (start 143.55 84.525) (end 143.675 84.65) (width 0.3048) (layer "F.Cu") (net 17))
 (via (at 143.55 82.3) (size 0.6096) (drill 0.3048) (layers "F.Cu" "B.Cu") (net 17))
 (via (at 136.089711 78.360289) (size 0.6096) (drill 0.3048) (layers "F.Cu" "B.Cu") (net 17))
 (segment (start 143.55 82.3) (end 142.4 81.15) (width 0.3048) (layer "B.Cu") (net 17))
 (segment (start 136.110289 78.360289) (end 136.089711 78.360289) (width 0.3048) (layer "B.Cu") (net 17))
 (segment (start 138.9 81.15) (end 136.110289 78.360289) (width 0.3048) (layer "B.Cu") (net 17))
 (segment (start 142.4 81.15) (end 138.9 81.15) (width 0.3048) (layer "B.Cu") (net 17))
 (segment (start 142.65 83.05) (end 142.425 83.275) (width 0.3048) (layer "F.Cu") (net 18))
 (segment (start 142.425 83.275) (end 142.425 84.65) (width 0.3048) (layer "F.Cu") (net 18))
 (segment (start 137.6 76.555) (end 137.6 78.35) (width 0.3048) (layer "F.Cu") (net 18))
 (via (at 142.65 83.05) (size 0.6096) (drill 0.3048) (layers "F.Cu" "B.Cu") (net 18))
 (via (at 137.6 78.35) (size 0.6096) (drill 0.3048) (layers "F.Cu" "B.Cu") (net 18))
 (segment (start 142.65 83.05) (end 143.9 83.05) (width 0.3048) (layer "B.Cu") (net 18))
 (segment (start 143.9 83.05) (end 144.5 82.45) (width 0.3048) (layer "B.Cu") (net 18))
 (segment (start 144.5 82.45) (end 144.5 81.770578) (width 0.3048) (layer "B.Cu") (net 18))
 (segment (start 143.079422 80.35) (end 139.6 80.35) (width 0.3048) (layer "B.Cu") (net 18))
 (segment (start 144.5 81.770578) (end 143.079422 80.35) (width 0.3048) (layer "B.Cu") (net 18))
 (segment (start 139.6 80.35) (end 137.6 78.35) (width 0.3048) (layer "B.Cu") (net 18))
 (segment (start 138.6 84.575) (end 138.675 84.65) (width 0.3048) (layer "F.Cu") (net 19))
 (segment (start 139.2 76.555) (end 139.2 78.15) (width 0.3048) (layer "F.Cu") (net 19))
 (segment (start 139.2 78.15) (end 139.25 78.2) (width 0.3048) (layer "F.Cu") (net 19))
 (segment (start 138.6 82.885852) (end 138.6 84.575) (width 0.3048) (layer "F.Cu") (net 19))
 (via (at 138.6 82.885852) (size 0.6096) (drill 0.3048) (layers "F.Cu" "B.Cu") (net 19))
 (via (at 139.25 78.2) (size 0.6096) (drill 0.3048) (layers "F.Cu" "B.Cu") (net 19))
 (segment (start 135.2 79.5) (end 135.2 78.1) (width 0.3048) (layer "B.Cu") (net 19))
 (segment (start 135.9 77.4) (end 138.45 77.4) (width 0.3048) (layer "B.Cu") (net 19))
 (segment (start 138.6 82.885852) (end 138.585852 82.885852) (width 0.3048) (layer "B.Cu") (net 19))
 (segment (start 135.2 78.1) (end 135.9 77.4) (width 0.3048) (layer "B.Cu") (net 19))
 (segment (start 138.585852 82.885852) (end 135.2 79.5) (width 0.3048) (layer "B.Cu") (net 19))
 (segment (start 138.45 77.4) (end 139.25 78.2) (width 0.3048) (layer "B.Cu") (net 19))
 (segment (start 138.35 61.7) (end 138.35 63.395) (width 0.3048) (layer "F.Cu") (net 20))
 (segment (start 138.35 63.395) (end 138.4 63.445) (width 0.3048) (layer "F.Cu") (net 20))
 (segment (start 141.314711 83.114711) (end 141.314711 84.510289) (width 0.3048) (layer "F.Cu") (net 20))
 (segment (start 141.314711 84.510289) (end 141.175 84.65) (width 0.3048) (layer "F.Cu") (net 20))
 (via (at 138.35 61.7) (size 0.6096) (drill 0.3048) (layers "F.Cu" "B.Cu") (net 20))
 (via (at 141.314711 83.114711) (size 0.6096) (drill 0.3048) (layers "F.Cu" "B.Cu") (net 20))
 (segment (start 134.5072 80.2072) (end 134.5072 63.1072) (width 0.3048) (layer "B.Cu") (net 20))
 (segment (start 133.6428 61.427778) (end 134.120578 60.95) (width 0.3048) (layer "B.Cu") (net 20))
 (segment (start 134.120578 60.95) (end 137.6 60.95) (width 0.3048) (layer "B.Cu") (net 20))
 (segment (start 140.88637 83.543052) (end 137.843052 83.543052) (width 0.3048) (layer "B.Cu") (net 20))
 (segment (start 134.5072 63.1072) (end 133.6428 62.2428) (width 0.3048) (layer "B.Cu") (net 20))
 (segment (start 137.6 60.95) (end 138.35 61.7) (width 0.3048) (layer "B.Cu") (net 20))
 (segment (start 137.843052 83.543052) (end 134.5072 80.2072) (width 0.3048) (layer "B.Cu") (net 20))
 (segment (start 141.314711 83.114711) (end 140.88637 83.543052) (width 0.3048) (layer "B.Cu") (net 20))
 (segment (start 133.6428 62.2428) (end 133.6428 61.427778) (width 0.3048) (layer "B.Cu") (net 20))
 (segment (start 135.4 61.65) (end 136 62.25) (width 0.3048) (layer "F.Cu") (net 21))
 (segment (start 147.425 83.775) (end 147.425 84.65) (width 0.3048) (layer "F.Cu") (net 21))
 (segment (start 148.3 82.9) (end 147.425 83.775) (width 0.3048) (layer "F.Cu") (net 21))
 (segment (start 136 62.25) (end 136 63.445) (width 0.3048) (layer "F.Cu") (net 21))
 (via (at 135.4 61.65) (size 0.6096) (drill 0.3048) (layers "F.Cu" "B.Cu") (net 21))
 (via (at 148.3 82.9) (size 0.6096) (drill 0.3048) (layers "F.Cu" "B.Cu") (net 21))
 (segment (start 136 70) (end 148.3 82.3) (width 0.3048) (layer "B.Cu") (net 21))
 (segment (start 148.3 82.3) (end 148.3 82.9) (width 0.3048) (layer "B.Cu") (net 21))
 (segment (start 136 62.25) (end 136 70) (width 0.3048) (layer "B.Cu") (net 21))
 (segment (start 135.4 61.65) (end 136 62.25) (width 0.3048) (layer "B.Cu") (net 21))
 (segment (start 146.95 82.95) (end 146.175 83.725) (width 0.3048) (layer "F.Cu") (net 22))
 (segment (start 135.2 63.445) (end 135.2 62.6) (width 0.3048) (layer "F.Cu") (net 22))
 (segment (start 146.175 83.725) (end 146.175 84.65) (width 0.3048) (layer "F.Cu") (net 22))
 (segment (start 135.2 62.6) (end 134.3 61.7) (width 0.3048) (layer "F.Cu") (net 22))
 (via (at 134.3 61.7) (size 0.6096) (drill 0.3048) (layers "F.Cu" "B.Cu") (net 22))
 (via (at 146.95 82.95) (size 0.6096) (drill 0.3048) (layers "F.Cu" "B.Cu") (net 22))
 (segment (start 146.95 81.9) (end 146.95 82.95) (width 0.3048) (layer "B.Cu") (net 22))
 (segment (start 135.2 62.6) (end 135.2 70.15) (width 0.3048) (layer "B.Cu") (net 22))
 (segment (start 135.2 70.15) (end 146.95 81.9) (width 0.3048) (layer "B.Cu") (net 22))
 (segment (start 134.3 61.7) (end 135.2 62.6) (width 0.3048) (layer "B.Cu") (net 22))
 (segment (start 150.275 84.3) (end 150.275 80.8) (width 0.3048) (layer "F.Cu") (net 14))
 (segment (start 149.925 84.65) (end 149.9 84.65) (width 0.3048) (layer "F.Cu") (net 14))
 (segment (start 149.925 84.65) (end 150.275 84.3) (width 0.3048) (layer "F.Cu") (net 14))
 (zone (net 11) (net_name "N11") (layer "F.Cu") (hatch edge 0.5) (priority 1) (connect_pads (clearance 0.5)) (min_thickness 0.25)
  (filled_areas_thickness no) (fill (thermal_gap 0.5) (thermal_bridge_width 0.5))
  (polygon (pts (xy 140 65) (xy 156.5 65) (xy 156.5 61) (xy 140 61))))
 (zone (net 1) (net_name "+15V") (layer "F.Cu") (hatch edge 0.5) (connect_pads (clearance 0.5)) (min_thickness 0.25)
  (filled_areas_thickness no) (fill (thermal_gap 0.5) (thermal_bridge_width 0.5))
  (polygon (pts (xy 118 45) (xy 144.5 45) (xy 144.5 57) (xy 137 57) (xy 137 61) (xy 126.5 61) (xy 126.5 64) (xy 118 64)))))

